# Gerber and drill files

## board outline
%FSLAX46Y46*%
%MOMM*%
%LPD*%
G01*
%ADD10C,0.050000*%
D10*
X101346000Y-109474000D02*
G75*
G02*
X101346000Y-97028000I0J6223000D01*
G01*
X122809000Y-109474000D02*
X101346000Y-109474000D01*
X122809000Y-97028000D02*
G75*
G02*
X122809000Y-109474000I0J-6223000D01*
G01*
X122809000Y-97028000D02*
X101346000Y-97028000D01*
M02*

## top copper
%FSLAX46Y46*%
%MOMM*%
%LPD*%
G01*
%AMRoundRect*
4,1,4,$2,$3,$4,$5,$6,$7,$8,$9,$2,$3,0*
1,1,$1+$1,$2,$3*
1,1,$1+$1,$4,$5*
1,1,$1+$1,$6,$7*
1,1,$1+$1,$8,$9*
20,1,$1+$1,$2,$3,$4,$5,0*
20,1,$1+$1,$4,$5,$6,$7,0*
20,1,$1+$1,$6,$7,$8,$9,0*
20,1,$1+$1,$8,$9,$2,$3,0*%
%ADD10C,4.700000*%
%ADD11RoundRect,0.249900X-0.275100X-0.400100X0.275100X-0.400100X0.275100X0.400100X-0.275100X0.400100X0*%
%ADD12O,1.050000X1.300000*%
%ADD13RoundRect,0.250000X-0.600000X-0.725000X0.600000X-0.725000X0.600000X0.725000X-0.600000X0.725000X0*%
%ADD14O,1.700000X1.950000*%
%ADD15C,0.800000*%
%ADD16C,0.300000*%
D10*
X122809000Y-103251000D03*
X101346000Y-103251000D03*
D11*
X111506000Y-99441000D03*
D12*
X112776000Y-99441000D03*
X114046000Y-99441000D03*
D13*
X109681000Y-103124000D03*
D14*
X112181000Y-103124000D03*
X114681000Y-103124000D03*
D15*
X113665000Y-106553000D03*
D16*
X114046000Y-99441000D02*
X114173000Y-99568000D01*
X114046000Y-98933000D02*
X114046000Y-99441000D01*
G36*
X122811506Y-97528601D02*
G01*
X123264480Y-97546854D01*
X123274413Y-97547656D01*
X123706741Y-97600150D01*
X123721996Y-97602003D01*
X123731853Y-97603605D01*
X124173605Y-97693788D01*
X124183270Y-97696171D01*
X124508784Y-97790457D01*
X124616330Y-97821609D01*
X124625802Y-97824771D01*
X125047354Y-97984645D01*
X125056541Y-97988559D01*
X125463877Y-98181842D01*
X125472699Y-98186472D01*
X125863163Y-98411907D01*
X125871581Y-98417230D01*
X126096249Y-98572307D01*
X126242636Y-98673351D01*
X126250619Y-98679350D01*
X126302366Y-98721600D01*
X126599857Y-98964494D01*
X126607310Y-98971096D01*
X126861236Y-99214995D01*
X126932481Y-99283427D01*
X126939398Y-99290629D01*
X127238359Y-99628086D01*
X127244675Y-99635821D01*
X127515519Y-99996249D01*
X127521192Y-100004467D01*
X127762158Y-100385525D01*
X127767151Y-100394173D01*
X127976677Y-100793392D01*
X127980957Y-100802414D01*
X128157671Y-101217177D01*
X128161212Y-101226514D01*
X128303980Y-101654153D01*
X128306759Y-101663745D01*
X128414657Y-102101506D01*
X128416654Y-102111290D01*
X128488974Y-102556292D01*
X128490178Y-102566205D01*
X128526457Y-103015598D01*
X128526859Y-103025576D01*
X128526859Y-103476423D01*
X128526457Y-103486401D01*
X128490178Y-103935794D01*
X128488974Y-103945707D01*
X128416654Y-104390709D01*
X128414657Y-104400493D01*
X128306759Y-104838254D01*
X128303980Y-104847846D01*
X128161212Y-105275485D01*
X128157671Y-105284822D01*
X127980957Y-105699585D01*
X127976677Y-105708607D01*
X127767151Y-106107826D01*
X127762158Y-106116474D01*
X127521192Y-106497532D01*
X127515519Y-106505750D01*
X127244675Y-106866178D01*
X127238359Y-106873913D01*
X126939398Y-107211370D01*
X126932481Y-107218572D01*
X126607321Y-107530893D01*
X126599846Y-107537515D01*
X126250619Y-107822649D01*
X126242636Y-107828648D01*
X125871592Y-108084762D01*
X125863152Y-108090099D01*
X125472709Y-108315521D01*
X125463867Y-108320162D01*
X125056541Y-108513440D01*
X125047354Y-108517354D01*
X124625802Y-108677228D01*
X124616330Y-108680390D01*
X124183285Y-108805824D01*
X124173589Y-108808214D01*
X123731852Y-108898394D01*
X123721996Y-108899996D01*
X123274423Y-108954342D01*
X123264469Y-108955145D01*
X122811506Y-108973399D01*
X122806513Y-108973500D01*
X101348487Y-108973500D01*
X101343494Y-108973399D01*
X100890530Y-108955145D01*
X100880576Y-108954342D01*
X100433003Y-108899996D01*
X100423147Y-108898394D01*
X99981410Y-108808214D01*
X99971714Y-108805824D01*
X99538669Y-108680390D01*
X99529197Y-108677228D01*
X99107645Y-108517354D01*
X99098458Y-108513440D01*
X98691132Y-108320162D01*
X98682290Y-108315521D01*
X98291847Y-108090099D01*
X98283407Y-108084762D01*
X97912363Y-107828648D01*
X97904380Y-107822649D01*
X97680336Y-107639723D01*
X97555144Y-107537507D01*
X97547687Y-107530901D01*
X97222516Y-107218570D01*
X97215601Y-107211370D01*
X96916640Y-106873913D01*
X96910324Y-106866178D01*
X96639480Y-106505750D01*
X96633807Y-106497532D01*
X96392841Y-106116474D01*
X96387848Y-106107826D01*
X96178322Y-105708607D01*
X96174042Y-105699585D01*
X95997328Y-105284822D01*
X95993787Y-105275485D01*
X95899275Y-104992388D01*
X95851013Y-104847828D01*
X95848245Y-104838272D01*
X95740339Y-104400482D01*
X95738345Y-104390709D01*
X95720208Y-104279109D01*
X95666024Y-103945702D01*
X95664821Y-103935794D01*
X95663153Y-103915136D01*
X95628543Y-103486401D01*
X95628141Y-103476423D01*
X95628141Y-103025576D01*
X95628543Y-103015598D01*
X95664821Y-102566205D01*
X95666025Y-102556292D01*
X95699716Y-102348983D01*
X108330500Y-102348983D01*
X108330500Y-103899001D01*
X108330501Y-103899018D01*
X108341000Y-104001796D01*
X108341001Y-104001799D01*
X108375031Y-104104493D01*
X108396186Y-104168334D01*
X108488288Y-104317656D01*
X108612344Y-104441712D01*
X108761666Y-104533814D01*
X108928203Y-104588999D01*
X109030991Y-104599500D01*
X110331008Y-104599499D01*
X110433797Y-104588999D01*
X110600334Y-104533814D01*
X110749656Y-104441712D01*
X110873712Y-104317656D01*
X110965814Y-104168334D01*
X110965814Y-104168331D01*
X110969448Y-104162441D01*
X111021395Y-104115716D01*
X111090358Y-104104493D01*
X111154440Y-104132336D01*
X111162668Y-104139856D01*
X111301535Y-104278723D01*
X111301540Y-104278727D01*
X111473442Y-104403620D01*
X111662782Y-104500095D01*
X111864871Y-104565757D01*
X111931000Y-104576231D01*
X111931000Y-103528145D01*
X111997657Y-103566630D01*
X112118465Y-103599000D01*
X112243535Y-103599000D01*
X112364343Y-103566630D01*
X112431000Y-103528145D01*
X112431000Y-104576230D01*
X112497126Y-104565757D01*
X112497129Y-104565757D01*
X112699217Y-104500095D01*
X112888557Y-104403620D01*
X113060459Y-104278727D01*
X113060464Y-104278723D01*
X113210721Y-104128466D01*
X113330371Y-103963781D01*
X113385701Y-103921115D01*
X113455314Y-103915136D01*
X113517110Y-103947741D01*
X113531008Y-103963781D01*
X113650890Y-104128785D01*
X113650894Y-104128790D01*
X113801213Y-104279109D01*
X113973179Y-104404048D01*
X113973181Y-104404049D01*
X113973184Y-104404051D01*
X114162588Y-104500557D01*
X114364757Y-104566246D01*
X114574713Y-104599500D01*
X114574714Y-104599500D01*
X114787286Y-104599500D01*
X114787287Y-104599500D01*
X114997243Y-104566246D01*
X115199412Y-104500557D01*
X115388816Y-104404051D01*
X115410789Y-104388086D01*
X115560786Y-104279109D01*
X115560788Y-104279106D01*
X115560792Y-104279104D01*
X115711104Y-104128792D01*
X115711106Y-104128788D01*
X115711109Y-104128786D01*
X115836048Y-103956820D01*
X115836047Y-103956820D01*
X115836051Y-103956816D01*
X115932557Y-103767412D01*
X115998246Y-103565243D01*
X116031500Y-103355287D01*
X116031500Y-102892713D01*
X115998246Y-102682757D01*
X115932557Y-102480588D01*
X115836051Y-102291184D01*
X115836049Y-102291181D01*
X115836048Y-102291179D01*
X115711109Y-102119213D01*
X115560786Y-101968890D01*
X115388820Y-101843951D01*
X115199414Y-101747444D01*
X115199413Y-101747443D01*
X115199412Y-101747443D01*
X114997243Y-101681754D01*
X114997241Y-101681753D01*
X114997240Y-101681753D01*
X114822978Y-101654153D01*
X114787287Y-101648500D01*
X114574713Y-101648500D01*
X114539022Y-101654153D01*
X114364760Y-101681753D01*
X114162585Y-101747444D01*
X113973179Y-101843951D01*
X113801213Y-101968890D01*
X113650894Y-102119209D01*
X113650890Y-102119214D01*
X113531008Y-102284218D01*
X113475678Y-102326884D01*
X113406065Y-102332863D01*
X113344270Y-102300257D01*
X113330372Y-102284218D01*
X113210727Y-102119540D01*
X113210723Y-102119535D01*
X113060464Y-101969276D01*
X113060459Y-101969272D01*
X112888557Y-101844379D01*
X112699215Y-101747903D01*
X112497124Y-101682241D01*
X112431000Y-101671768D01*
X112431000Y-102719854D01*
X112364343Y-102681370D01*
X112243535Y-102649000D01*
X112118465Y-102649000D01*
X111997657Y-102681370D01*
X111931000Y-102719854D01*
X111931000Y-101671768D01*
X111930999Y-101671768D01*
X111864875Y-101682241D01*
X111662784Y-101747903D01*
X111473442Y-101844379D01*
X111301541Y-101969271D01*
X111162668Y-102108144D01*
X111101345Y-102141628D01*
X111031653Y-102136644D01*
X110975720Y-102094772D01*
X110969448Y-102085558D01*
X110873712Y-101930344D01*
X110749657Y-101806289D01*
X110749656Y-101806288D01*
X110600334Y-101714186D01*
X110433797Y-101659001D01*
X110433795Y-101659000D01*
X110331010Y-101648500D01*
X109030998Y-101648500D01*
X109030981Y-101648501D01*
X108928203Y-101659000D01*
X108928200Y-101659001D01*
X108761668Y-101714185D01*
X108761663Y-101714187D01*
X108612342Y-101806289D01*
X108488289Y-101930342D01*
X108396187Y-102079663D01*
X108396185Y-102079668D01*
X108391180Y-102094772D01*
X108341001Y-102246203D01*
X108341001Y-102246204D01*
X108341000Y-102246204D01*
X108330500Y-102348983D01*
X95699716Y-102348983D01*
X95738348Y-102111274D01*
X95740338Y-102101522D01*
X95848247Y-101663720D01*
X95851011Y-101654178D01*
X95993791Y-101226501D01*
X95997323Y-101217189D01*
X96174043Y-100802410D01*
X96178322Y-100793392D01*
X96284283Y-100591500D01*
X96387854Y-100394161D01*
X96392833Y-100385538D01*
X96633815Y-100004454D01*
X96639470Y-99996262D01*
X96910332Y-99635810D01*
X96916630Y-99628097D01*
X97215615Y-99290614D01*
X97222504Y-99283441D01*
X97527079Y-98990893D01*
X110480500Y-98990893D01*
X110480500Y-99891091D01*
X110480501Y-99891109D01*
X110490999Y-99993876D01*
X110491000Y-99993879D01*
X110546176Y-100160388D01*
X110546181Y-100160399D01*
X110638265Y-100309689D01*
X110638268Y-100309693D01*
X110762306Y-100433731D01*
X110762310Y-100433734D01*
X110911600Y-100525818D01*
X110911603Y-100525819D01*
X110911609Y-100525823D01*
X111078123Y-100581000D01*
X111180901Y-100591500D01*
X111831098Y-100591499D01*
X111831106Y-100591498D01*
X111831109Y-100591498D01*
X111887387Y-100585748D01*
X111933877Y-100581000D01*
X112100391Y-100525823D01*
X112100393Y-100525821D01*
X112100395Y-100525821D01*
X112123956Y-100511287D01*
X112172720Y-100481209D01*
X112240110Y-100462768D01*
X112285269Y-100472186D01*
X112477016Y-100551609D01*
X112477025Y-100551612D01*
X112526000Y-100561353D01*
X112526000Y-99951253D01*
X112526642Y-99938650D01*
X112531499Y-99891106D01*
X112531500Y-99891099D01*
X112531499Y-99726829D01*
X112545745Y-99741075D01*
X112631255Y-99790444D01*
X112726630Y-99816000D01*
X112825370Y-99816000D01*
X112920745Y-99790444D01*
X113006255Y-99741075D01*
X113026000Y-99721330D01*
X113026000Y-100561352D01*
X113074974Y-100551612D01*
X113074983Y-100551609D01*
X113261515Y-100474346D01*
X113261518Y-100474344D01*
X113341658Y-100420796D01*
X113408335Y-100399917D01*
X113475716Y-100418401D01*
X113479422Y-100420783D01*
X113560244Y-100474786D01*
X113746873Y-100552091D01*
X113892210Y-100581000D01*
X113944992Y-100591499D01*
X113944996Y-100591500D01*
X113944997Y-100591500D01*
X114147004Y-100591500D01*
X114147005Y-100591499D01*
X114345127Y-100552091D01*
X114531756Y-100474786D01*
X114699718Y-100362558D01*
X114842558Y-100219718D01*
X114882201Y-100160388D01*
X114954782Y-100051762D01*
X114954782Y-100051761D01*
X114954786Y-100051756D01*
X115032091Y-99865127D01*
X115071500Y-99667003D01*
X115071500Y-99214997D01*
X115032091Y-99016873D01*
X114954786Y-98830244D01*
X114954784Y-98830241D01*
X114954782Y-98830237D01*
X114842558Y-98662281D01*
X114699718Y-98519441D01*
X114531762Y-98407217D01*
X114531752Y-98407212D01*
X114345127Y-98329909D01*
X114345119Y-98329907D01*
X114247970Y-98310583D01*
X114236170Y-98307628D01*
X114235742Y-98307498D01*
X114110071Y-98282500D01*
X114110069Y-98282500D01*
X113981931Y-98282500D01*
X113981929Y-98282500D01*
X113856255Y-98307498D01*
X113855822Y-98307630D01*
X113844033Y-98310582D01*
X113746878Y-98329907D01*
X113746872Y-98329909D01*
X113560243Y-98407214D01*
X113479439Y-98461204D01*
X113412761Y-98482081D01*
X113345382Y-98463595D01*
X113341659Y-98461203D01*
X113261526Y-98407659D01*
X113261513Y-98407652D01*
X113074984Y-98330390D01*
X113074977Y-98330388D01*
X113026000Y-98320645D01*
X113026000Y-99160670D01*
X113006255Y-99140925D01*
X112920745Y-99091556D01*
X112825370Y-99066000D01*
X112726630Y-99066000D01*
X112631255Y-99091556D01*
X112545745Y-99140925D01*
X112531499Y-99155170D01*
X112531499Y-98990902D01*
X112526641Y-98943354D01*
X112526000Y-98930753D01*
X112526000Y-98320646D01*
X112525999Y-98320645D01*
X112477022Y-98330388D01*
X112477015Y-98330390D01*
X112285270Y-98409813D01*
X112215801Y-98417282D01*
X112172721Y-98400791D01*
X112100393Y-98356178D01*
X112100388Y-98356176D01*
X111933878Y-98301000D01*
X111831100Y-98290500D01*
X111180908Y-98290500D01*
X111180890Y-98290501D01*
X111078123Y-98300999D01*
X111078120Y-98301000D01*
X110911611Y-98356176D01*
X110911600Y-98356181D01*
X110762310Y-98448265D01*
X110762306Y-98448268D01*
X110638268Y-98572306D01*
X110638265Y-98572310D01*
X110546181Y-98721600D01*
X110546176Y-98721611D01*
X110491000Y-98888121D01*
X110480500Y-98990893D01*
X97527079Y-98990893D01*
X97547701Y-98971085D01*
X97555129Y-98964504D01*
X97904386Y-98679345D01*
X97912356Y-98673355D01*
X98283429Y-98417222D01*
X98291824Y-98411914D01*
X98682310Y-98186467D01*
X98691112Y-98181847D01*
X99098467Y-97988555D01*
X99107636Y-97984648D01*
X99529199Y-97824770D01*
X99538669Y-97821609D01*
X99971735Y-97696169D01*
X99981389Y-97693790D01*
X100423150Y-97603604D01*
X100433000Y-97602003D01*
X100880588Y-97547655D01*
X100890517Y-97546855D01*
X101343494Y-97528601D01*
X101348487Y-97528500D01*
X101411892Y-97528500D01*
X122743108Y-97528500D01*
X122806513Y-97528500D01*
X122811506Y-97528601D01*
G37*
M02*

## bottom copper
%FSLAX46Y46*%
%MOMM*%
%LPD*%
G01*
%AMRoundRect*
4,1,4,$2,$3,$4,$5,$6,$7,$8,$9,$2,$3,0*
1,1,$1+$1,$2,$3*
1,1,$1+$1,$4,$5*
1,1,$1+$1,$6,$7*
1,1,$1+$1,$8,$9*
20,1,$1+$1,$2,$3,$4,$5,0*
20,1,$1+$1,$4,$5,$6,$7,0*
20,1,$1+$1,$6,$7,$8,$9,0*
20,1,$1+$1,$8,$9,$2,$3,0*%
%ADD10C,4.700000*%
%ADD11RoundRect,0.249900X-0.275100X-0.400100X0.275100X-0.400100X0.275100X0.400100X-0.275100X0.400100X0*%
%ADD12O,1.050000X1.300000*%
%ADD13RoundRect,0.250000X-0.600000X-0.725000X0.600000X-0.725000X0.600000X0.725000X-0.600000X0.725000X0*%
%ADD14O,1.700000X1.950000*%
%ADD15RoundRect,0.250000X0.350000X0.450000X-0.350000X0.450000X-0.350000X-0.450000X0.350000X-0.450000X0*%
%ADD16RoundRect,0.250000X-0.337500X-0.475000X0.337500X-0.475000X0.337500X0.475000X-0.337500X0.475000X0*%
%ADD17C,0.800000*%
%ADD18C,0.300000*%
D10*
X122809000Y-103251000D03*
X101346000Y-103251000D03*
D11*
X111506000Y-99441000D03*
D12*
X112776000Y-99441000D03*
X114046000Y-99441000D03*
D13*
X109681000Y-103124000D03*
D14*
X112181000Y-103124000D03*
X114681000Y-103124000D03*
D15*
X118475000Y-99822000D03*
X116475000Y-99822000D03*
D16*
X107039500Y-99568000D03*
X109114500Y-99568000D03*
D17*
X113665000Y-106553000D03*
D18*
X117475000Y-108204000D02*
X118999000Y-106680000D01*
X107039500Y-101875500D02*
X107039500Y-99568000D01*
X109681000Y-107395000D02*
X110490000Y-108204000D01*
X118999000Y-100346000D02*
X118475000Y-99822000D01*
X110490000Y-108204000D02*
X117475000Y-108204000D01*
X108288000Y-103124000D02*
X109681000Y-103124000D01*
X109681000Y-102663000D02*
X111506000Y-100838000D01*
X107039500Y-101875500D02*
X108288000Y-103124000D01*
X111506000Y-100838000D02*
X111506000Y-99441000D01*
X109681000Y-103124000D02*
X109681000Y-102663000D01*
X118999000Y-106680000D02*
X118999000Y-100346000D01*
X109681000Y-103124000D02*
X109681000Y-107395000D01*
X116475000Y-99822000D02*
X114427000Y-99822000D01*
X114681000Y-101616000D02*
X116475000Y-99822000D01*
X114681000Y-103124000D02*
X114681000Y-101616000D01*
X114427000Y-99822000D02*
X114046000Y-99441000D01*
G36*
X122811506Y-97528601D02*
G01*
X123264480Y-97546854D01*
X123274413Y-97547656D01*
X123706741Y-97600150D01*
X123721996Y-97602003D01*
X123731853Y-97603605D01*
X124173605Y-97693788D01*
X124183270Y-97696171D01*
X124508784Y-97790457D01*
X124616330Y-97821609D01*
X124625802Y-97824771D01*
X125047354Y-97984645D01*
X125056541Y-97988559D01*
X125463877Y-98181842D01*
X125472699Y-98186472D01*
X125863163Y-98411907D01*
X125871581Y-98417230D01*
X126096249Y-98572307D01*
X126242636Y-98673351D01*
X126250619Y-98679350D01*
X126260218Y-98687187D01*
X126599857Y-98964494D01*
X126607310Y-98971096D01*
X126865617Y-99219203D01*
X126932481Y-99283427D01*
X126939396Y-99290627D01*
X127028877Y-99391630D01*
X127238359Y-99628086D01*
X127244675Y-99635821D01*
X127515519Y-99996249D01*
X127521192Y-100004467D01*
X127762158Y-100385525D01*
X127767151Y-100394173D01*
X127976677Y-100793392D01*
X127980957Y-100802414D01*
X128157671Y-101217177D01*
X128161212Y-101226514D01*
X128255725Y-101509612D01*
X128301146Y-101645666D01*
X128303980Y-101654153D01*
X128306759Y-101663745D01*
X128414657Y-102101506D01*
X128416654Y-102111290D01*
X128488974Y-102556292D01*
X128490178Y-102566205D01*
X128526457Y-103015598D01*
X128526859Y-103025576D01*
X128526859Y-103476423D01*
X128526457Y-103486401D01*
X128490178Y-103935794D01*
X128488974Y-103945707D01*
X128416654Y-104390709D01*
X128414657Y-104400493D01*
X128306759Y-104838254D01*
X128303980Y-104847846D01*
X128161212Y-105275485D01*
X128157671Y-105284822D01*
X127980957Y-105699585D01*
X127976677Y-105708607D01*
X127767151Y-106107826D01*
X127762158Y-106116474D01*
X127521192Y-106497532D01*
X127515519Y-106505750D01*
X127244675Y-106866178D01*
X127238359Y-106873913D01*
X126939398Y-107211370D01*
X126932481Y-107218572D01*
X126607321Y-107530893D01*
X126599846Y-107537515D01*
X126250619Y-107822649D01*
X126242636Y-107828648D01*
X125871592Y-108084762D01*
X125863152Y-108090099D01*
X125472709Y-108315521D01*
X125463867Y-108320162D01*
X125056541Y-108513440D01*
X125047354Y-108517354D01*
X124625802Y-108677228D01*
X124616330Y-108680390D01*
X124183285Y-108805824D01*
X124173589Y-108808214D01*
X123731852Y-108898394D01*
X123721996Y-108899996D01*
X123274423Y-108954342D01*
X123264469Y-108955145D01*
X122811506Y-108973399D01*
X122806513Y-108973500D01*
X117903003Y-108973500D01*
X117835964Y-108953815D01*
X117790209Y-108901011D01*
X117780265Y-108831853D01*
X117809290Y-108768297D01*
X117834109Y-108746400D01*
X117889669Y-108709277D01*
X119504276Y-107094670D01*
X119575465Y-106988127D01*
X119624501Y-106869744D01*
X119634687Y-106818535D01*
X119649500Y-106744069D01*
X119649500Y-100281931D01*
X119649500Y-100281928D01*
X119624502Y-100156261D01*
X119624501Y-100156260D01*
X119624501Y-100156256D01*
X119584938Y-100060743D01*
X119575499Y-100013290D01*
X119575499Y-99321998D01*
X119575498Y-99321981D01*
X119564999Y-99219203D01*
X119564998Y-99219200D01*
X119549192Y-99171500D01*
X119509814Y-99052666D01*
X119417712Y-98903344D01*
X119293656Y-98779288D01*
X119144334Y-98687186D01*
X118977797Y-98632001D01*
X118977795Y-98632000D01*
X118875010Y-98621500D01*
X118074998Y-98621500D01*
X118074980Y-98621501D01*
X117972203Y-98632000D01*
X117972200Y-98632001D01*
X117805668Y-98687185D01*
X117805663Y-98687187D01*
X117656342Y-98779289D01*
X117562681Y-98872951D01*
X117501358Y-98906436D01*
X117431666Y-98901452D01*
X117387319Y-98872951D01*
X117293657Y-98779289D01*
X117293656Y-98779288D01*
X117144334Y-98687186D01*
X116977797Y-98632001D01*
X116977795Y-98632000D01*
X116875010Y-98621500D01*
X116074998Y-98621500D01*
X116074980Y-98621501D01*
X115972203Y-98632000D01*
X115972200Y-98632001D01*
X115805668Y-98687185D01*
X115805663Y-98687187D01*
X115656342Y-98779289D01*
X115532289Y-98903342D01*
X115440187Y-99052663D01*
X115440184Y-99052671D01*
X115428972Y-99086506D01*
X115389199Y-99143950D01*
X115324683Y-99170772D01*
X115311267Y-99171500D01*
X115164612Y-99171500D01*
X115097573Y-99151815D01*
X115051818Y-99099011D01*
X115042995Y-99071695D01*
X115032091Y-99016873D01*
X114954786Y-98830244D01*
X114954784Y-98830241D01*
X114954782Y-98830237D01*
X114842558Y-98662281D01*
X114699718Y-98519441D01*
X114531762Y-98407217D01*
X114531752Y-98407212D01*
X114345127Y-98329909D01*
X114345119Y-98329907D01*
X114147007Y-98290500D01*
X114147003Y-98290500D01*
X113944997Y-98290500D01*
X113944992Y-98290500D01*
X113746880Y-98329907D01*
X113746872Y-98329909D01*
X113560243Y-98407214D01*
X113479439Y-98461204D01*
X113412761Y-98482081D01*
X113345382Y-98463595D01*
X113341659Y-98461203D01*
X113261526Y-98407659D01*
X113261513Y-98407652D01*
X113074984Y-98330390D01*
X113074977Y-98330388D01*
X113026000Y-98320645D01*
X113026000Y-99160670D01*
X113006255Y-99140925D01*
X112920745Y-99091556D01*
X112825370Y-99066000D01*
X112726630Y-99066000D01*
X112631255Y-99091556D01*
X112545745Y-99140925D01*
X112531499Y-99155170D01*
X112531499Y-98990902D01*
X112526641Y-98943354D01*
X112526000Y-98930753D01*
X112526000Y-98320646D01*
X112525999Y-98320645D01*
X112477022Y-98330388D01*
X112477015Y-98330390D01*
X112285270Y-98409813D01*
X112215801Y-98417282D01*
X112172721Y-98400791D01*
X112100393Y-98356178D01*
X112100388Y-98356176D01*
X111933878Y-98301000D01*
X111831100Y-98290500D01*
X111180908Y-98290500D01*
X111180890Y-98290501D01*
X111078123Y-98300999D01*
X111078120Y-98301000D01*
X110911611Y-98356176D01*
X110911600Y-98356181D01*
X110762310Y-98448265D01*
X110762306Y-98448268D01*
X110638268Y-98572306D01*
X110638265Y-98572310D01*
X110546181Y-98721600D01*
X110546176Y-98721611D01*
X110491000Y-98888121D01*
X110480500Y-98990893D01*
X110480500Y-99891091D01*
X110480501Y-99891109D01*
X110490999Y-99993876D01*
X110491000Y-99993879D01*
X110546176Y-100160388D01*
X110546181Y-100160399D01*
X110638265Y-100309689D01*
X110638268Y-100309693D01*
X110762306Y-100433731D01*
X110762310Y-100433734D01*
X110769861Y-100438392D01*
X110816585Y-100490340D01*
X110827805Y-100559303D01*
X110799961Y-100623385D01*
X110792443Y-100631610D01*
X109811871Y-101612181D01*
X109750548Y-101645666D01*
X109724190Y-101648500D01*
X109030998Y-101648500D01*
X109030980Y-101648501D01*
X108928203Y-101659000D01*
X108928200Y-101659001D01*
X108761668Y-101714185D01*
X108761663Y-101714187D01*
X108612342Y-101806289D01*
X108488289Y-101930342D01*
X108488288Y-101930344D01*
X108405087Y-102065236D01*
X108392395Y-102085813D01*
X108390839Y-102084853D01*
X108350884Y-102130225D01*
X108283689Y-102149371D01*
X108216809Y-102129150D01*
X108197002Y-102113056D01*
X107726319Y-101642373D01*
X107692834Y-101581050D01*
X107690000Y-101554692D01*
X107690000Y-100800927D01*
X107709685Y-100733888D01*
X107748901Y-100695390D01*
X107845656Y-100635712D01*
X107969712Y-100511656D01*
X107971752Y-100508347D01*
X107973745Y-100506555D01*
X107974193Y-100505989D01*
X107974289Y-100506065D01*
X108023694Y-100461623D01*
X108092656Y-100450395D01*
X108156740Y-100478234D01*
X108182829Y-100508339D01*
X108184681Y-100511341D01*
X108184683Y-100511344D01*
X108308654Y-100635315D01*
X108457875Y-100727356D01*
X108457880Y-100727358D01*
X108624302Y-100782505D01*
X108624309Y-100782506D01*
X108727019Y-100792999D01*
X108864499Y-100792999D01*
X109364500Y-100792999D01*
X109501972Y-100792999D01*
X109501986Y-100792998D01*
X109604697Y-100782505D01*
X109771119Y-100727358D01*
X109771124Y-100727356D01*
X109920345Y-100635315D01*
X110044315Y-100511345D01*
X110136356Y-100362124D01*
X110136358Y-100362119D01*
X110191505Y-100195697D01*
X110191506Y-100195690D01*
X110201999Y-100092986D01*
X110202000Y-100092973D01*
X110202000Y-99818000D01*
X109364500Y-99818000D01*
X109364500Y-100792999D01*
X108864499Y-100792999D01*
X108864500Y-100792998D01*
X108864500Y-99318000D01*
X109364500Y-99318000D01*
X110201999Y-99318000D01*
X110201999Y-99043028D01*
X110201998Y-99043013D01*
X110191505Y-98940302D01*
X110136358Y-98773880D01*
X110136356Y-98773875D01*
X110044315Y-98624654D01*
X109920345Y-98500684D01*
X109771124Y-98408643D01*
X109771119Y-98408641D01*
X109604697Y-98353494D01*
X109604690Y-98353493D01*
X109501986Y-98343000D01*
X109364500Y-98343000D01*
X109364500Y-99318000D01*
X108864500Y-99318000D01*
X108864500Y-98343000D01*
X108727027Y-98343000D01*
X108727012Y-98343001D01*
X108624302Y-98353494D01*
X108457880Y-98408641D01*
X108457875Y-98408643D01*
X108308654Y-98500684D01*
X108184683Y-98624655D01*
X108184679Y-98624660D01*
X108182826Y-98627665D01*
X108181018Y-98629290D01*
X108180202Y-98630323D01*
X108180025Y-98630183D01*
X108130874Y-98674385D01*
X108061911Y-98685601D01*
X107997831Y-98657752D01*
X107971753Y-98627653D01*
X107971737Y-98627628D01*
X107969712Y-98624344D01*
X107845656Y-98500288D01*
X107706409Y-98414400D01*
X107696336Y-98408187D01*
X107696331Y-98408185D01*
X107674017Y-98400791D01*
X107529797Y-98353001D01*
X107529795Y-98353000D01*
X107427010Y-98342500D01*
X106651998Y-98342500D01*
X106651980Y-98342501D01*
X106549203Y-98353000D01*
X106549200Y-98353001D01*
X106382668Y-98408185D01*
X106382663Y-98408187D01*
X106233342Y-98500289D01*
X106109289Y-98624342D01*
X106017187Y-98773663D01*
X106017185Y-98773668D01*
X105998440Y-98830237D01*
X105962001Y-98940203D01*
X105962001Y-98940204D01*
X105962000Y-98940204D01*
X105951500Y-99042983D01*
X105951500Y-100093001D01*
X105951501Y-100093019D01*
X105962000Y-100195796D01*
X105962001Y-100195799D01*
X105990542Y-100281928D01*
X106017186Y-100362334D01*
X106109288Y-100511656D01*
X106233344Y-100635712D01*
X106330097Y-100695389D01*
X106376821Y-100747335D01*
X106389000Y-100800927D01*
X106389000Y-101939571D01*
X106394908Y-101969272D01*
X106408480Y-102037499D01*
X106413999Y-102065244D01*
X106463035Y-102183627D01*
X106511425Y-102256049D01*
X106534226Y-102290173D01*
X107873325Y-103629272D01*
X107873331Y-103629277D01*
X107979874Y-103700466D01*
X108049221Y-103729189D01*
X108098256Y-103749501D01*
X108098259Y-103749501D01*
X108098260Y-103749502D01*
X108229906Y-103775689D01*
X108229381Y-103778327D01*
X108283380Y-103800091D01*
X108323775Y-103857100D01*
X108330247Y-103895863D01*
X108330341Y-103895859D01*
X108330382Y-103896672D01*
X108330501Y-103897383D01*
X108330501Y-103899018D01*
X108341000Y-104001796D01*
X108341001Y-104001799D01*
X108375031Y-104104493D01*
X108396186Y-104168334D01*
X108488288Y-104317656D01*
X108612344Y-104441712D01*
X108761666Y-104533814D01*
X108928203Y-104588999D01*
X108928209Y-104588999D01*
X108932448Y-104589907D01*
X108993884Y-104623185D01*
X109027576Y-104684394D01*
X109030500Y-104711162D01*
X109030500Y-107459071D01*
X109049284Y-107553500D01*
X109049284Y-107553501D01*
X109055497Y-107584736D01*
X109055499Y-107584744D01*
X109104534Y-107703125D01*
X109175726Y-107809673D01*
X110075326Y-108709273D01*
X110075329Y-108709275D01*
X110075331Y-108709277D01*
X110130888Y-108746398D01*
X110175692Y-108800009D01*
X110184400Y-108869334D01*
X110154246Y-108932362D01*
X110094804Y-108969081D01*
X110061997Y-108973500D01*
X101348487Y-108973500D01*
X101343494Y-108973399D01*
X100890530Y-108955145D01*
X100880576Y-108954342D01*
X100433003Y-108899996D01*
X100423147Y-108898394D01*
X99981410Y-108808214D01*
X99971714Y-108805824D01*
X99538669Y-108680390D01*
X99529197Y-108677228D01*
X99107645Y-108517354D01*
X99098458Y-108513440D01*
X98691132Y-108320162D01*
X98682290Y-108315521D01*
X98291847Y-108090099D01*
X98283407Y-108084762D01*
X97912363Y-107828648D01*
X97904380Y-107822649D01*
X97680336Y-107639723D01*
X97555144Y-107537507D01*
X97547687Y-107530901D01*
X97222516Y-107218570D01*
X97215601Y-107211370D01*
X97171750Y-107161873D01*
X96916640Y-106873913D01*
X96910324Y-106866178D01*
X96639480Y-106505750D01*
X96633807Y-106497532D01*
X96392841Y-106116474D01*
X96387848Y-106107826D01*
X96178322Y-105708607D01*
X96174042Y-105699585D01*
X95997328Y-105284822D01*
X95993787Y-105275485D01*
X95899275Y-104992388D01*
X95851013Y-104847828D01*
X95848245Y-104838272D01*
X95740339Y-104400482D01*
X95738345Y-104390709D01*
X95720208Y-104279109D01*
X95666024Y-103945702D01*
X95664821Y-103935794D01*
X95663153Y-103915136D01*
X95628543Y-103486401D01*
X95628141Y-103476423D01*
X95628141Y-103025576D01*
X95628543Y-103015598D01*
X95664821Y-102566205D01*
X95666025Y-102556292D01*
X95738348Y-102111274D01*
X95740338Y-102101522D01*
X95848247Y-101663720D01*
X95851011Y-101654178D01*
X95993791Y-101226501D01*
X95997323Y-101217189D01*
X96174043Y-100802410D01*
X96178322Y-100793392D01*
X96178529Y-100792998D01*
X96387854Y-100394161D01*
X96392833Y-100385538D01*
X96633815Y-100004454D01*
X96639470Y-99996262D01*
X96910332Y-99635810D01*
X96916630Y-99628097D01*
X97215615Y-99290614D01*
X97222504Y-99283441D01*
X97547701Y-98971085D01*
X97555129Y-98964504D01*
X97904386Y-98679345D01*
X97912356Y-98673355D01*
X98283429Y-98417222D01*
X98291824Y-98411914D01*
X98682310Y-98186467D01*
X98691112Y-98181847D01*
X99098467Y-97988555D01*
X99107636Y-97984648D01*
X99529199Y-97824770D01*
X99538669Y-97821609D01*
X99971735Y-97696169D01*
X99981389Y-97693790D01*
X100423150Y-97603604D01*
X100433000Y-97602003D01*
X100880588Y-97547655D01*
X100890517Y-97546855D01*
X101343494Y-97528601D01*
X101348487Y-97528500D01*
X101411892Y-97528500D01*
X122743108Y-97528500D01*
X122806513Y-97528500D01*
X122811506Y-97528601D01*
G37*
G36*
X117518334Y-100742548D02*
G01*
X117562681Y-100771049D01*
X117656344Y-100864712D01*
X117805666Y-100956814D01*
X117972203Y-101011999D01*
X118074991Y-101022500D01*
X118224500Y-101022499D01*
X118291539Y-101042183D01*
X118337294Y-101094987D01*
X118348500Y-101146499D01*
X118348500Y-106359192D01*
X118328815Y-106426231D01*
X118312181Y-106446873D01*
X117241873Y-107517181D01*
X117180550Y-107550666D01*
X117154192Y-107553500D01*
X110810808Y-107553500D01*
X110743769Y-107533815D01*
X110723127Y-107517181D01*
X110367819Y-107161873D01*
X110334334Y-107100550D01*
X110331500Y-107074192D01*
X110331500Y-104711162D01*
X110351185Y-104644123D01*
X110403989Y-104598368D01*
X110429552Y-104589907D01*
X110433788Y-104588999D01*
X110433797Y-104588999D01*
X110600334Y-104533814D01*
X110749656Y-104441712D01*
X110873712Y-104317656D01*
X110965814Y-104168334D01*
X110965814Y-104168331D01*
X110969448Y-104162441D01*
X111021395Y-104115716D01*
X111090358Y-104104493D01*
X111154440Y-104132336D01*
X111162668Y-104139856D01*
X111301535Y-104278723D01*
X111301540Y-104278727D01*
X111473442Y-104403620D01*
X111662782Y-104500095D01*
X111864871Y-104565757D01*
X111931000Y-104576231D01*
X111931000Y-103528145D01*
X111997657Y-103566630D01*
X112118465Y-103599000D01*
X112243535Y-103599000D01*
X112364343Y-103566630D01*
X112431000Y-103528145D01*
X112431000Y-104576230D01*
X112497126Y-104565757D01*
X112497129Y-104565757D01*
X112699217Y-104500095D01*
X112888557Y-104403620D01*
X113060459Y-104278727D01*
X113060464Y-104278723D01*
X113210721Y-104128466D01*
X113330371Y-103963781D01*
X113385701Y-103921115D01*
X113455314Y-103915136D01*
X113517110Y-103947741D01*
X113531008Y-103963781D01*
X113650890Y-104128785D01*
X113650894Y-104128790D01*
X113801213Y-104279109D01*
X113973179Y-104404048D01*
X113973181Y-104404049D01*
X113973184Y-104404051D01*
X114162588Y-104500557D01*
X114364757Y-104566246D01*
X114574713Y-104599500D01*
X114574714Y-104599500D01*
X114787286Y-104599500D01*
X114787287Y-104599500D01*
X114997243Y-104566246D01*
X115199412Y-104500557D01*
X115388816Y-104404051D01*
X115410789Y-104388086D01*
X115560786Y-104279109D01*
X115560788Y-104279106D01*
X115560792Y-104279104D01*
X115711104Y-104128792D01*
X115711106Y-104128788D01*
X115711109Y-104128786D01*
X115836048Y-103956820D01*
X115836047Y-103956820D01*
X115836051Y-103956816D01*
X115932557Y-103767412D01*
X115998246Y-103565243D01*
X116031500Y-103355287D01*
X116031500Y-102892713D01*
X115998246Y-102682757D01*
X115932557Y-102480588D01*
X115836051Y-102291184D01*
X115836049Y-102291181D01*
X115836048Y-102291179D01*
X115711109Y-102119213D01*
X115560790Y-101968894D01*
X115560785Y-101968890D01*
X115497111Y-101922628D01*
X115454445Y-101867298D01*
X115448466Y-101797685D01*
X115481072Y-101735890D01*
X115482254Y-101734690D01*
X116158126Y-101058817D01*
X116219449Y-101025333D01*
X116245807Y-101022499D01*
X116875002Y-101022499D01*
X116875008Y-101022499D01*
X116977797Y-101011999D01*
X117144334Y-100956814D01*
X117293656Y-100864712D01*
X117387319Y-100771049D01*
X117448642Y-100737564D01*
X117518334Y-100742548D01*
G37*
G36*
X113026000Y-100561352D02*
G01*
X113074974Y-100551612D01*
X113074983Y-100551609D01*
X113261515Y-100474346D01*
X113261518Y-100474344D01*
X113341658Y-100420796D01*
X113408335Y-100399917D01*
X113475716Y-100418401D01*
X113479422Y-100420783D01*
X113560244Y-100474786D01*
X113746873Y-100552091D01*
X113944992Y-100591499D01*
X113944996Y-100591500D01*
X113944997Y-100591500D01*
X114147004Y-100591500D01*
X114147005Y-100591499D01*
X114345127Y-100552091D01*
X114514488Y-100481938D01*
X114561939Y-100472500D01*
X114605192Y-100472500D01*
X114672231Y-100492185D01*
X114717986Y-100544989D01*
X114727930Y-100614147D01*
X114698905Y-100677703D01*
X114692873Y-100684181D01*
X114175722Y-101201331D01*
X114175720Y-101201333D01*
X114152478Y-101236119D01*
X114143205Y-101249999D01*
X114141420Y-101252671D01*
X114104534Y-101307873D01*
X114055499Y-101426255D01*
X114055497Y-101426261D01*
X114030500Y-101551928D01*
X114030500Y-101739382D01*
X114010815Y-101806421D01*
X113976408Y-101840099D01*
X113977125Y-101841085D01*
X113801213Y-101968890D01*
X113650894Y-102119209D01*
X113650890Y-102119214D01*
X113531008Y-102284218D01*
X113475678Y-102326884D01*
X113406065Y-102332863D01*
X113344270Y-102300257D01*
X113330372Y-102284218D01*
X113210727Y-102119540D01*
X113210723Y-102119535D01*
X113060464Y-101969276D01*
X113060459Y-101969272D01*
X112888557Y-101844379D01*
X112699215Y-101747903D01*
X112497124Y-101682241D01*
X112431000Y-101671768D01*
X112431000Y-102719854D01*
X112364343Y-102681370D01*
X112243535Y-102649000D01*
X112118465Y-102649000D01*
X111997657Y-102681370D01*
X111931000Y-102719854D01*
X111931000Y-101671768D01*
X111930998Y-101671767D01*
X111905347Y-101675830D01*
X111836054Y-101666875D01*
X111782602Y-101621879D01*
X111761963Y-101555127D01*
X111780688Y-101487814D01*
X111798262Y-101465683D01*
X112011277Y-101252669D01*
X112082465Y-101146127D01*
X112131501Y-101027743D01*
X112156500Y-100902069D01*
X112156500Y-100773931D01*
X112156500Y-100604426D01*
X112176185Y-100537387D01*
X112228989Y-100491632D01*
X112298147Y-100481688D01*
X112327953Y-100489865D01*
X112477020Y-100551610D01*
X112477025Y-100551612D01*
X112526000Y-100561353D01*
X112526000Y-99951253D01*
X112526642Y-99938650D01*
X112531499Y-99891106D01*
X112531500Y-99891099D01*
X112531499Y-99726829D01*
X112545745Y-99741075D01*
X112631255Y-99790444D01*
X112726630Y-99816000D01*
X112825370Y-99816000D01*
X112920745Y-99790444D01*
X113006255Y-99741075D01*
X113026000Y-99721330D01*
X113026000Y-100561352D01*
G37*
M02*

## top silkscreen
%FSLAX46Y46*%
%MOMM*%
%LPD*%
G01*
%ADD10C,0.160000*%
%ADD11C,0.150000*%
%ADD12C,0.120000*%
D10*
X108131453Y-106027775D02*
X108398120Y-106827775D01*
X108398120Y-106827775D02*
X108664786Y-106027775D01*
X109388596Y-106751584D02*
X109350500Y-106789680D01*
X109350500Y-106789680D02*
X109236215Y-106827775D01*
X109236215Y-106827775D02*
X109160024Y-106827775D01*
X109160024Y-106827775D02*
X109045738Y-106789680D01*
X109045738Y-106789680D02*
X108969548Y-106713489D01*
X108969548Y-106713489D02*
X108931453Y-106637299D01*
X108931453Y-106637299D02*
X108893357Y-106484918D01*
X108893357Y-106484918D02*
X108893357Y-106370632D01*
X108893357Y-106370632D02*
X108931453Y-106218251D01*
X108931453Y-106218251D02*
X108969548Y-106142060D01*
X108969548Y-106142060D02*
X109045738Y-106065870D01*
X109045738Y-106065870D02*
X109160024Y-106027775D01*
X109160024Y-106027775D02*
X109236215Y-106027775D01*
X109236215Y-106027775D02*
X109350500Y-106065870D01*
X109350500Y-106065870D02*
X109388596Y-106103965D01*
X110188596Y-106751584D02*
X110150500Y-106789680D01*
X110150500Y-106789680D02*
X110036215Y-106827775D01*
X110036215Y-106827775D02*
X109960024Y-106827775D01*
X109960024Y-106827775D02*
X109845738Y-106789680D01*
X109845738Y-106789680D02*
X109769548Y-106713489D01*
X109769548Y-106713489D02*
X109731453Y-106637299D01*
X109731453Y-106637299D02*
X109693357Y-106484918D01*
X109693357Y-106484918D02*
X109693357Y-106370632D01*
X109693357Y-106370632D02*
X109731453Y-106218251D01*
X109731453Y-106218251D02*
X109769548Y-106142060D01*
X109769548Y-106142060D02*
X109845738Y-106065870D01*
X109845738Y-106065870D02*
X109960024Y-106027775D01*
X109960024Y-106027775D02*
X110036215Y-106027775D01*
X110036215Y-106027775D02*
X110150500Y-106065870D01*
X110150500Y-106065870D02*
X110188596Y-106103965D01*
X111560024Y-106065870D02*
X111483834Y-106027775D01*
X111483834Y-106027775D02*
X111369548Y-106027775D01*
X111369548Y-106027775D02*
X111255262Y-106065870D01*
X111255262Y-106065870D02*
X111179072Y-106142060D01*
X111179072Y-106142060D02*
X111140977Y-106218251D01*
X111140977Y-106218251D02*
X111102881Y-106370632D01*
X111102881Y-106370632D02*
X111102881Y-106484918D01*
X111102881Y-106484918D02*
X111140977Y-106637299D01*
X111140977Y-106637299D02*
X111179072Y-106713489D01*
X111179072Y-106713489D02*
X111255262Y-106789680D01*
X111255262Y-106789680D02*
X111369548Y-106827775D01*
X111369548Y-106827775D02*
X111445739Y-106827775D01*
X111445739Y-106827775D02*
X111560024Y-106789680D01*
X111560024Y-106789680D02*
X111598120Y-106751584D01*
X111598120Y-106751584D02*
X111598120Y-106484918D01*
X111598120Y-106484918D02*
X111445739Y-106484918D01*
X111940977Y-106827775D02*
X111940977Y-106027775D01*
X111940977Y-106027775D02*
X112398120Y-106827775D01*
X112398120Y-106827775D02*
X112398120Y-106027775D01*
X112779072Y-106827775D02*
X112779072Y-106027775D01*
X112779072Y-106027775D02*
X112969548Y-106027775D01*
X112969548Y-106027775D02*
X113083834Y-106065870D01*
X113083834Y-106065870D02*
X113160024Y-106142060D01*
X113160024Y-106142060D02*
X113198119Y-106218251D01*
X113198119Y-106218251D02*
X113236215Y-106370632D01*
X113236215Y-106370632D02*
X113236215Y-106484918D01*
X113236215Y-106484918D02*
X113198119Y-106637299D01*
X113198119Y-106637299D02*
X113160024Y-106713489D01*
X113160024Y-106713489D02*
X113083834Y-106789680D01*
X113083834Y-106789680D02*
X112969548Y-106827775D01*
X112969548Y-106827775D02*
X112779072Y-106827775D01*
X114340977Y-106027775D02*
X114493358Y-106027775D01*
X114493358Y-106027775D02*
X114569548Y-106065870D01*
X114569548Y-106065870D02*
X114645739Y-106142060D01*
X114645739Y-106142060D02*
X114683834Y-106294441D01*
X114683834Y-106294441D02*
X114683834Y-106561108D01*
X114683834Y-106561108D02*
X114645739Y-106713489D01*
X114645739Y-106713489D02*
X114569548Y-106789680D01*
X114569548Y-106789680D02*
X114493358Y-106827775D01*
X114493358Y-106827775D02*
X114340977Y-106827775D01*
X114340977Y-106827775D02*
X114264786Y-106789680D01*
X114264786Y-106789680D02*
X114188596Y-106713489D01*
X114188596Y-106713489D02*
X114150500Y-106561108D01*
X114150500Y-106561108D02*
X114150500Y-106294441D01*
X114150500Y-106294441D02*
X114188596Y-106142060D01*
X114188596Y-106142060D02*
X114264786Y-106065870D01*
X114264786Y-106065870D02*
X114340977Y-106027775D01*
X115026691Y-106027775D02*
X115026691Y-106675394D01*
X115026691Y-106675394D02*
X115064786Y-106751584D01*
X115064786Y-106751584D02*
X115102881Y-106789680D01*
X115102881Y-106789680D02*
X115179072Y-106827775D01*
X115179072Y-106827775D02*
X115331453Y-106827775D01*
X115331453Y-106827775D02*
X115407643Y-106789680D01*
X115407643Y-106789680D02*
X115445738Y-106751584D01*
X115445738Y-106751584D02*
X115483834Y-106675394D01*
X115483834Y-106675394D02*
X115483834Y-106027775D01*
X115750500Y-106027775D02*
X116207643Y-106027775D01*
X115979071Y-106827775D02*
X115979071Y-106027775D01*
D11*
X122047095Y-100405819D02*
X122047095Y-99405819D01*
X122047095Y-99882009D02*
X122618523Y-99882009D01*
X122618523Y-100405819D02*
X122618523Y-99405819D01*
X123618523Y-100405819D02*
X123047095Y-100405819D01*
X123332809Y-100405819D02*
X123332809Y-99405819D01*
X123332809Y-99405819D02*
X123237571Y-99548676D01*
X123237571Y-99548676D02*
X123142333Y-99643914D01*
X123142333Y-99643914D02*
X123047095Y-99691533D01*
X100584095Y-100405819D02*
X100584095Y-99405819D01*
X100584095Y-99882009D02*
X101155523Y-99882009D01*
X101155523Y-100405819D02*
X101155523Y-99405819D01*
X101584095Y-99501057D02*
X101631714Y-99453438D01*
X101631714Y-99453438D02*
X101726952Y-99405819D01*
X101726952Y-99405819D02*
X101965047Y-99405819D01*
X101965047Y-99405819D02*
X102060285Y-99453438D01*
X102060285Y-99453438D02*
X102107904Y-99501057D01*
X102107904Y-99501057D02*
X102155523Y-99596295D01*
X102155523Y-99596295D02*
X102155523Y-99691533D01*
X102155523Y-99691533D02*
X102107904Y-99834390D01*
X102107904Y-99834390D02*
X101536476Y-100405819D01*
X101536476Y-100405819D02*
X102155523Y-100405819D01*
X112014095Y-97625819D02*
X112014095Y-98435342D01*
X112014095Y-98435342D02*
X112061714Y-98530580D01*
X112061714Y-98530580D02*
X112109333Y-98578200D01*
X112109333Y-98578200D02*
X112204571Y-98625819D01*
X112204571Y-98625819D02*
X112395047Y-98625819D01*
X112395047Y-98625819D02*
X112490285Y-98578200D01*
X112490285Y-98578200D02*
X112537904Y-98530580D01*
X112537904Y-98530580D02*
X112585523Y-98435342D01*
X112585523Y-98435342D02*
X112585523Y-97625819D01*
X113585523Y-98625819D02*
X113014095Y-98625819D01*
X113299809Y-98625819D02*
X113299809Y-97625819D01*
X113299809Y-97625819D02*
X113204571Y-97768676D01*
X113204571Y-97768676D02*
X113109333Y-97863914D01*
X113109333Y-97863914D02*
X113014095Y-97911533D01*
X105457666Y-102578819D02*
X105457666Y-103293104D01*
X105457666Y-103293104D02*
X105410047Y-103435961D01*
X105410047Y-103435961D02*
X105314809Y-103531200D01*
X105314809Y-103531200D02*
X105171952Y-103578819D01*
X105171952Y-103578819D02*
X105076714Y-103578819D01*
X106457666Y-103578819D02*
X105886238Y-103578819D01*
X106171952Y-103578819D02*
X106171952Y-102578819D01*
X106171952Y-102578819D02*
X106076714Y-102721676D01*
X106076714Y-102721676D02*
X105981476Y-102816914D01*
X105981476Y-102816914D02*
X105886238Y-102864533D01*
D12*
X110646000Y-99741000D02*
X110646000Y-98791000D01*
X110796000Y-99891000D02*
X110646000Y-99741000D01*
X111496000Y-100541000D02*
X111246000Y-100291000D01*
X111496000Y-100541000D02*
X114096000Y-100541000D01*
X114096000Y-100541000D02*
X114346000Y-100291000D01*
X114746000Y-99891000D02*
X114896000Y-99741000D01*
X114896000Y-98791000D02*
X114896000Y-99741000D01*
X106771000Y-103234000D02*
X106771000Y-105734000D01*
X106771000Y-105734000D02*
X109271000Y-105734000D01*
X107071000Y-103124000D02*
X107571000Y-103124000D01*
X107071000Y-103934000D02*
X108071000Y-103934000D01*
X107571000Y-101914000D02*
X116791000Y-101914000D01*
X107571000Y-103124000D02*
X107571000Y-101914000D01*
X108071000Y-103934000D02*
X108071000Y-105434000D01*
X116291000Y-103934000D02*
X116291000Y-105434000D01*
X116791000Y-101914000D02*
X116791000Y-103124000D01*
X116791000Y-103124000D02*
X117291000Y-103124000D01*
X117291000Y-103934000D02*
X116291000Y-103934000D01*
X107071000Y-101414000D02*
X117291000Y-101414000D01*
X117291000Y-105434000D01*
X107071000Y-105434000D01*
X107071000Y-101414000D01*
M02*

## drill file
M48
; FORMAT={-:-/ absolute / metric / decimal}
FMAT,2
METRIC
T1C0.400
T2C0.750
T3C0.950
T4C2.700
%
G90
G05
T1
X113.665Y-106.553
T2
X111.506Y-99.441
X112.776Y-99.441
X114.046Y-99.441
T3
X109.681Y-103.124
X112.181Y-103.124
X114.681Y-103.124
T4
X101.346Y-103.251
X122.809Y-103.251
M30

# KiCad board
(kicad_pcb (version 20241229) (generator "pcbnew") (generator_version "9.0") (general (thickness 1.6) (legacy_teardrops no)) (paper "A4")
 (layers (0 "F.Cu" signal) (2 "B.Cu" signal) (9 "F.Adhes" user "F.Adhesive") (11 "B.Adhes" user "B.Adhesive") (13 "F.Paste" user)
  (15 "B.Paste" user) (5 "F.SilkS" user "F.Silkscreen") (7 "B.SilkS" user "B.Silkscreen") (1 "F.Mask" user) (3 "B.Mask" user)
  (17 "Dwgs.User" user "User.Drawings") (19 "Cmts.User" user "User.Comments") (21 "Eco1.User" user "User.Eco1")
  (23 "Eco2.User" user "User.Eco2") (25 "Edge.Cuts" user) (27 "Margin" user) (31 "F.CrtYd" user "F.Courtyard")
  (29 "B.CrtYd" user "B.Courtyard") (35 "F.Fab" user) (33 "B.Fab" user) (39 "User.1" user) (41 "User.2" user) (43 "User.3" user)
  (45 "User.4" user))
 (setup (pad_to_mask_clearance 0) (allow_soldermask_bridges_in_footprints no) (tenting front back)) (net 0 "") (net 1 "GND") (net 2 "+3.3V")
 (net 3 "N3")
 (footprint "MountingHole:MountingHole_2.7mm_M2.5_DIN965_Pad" (layer "F.Cu") (at 122.809 103.251)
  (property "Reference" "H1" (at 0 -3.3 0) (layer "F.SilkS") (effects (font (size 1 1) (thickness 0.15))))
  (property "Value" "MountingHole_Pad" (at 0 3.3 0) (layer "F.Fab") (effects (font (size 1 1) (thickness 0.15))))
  (pad "1" thru_hole circle (at 0 0) (size 4.7 4.7) (drill 2.7) (layers "*.Cu" "*.Mask") (remove_unused_layers no) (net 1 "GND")
   (zone_connect 2)))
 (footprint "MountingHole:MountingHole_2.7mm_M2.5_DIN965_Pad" (layer "F.Cu") (at 101.346 103.251)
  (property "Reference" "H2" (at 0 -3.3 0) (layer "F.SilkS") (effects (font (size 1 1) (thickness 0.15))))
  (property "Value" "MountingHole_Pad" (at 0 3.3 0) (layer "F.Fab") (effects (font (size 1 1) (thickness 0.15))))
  (pad "1" thru_hole circle (at 0 0) (size 4.7 4.7) (drill 2.7) (layers "*.Cu" "*.Mask") (remove_unused_layers no) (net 1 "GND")
   (zone_connect 2)))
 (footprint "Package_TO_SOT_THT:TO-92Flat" (layer "F.Cu") (at 111.506 99.441)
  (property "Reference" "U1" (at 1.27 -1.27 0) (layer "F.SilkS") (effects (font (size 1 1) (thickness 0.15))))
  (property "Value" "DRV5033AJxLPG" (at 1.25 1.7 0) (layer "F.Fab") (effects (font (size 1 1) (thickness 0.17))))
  (fp_line (start -0.86 0.3) (end -0.86 -0.65) (stroke (width 0.12) (type solid)) (layer "F.SilkS"))
  (fp_line (start -0.71 0.45) (end -0.86 0.3) (stroke (width 0.12) (type solid)) (layer "F.SilkS"))
  (fp_line (start -0.01 1.1) (end -0.26 0.85) (stroke (width 0.12) (type solid)) (layer "F.SilkS"))
  (fp_line (start -0.01 1.1) (end 2.59 1.1) (stroke (width 0.12) (type solid)) (layer "F.SilkS"))
  (fp_line (start 2.59 1.1) (end 2.84 0.85) (stroke (width 0.12) (type solid)) (layer "F.SilkS"))
  (fp_line (start 3.24 0.45) (end 3.39 0.3) (stroke (width 0.12) (type solid)) (layer "F.SilkS"))
  (fp_line (start 3.39 -0.65) (end 3.39 0.3) (stroke (width 0.12) (type solid)) (layer "F.SilkS"))
  (pad "1" thru_hole roundrect (at 0 0) (size 1.05 1.3) (drill 0.75) (layers "*.Cu" "*.Mask") (remove_unused_layers no)
   (roundrect_rratio 0.238) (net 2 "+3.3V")
   (teardrops (best_length_ratio 0.5) (max_length 1) (best_width_ratio 1) (max_width 1) (curved_edges no) (filter_ratio 0.9) (enabled no)
    (allow_two_segments yes) (prefer_zone_connections yes)))
  (pad "2" thru_hole oval (at 1.27 0) (size 1.05 1.3) (drill 0.75) (layers "*.Cu" "*.Mask") (remove_unused_layers no) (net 1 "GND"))
  (pad "3" thru_hole oval (at 2.54 0) (size 1.05 1.3) (drill 0.75) (layers "*.Cu" "*.Mask") (remove_unused_layers no) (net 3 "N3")))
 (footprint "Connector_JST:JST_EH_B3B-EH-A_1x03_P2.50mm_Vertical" (layer "F.Cu") (at 109.681 103.124)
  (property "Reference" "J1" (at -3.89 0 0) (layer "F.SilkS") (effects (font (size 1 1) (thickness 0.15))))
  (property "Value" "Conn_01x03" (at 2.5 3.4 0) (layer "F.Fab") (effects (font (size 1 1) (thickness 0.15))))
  (fp_line (start -2.91 0.11) (end -2.91 2.61) (stroke (width 0.12) (type solid)) (layer "F.SilkS"))
  (fp_line (start -2.91 2.61) (end -0.41 2.61) (stroke (width 0.12) (type solid)) (layer "F.SilkS"))
  (fp_line (start -2.61 0) (end -2.11 0) (stroke (width 0.12) (type solid)) (layer "F.SilkS"))
  (fp_line (start -2.61 0.81) (end -1.61 0.81) (stroke (width 0.12) (type solid)) (layer "F.SilkS"))
  (fp_line (start -2.11 -1.21) (end 7.11 -1.21) (stroke (width 0.12) (type solid)) (layer "F.SilkS"))
  (fp_line (start -2.11 0) (end -2.11 -1.21) (stroke (width 0.12) (type solid)) (layer "F.SilkS"))
  (fp_line (start -1.61 0.81) (end -1.61 2.31) (stroke (width 0.12) (type solid)) (layer "F.SilkS"))
  (fp_line (start 6.61 0.81) (end 6.61 2.31) (stroke (width 0.12) (type solid)) (layer "F.SilkS"))
  (fp_line (start 7.11 -1.21) (end 7.11 0) (stroke (width 0.12) (type solid)) (layer "F.SilkS"))
  (fp_line (start 7.11 0) (end 7.61 0) (stroke (width 0.12) (type solid)) (layer "F.SilkS"))
  (fp_line (start 7.61 0.81) (end 6.61 0.81) (stroke (width 0.12) (type solid)) (layer "F.SilkS"))
  (fp_rect (start -2.61 -1.71) (end 7.61 2.31) (stroke (width 0.12) (type solid)) (fill no) (layer "F.SilkS"))
  (pad "1" thru_hole roundrect (at 0 0) (size 1.7 1.95) (drill 0.95) (layers "*.Cu" "*.Mask") (remove_unused_layers no)
   (roundrect_rratio 0.147059) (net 2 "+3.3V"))
  (pad "2" thru_hole oval (at 2.5 0) (size 1.7 1.95) (drill 0.95) (layers "*.Cu" "*.Mask") (remove_unused_layers no) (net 1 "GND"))
  (pad "3" thru_hole oval (at 5 0) (size 1.7 1.95) (drill 0.95) (layers "*.Cu" "*.Mask") (remove_unused_layers no) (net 3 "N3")))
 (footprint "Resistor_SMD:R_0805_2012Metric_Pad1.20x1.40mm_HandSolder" (layer "B.Cu") (at 117.475 99.822 180)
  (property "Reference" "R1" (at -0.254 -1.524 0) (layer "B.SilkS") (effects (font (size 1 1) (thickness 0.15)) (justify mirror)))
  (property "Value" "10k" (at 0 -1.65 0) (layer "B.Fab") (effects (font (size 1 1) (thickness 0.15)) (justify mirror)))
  (pad "1" smd roundrect (at -1 0 180) (size 1.2 1.4) (layers "B.Cu" "B.Mask" "B.Paste") (roundrect_rratio 0.208333) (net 2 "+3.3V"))
  (pad "2" smd roundrect (at 1 0 180) (size 1.2 1.4) (layers "B.Cu" "B.Mask" "B.Paste") (roundrect_rratio 0.208333) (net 3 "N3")))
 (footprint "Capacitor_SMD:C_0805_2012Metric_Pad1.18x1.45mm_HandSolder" (layer "B.Cu") (at 108.077 99.568)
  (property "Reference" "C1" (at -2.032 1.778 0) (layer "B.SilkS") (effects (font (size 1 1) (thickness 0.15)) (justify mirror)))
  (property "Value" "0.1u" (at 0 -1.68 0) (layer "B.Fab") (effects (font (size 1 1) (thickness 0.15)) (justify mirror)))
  (pad "1" smd roundrect (at -1.0375 0) (size 1.175 1.45) (layers "B.Cu" "B.Mask" "B.Paste") (roundrect_rratio 0.212766) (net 2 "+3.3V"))
  (pad "2" smd roundrect (at 1.0375 0) (size 1.175 1.45) (layers "B.Cu" "B.Mask" "B.Paste") (roundrect_rratio 0.212766) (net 1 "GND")))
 (gr_arc (start 101.346 109.474) (mid 95.123 103.251) (end 101.346 97.028) (stroke (width 0.05) (type default)) (layer "Edge.Cuts"))
 (gr_line (start 122.809 109.474) (end 101.346 109.474) (stroke (width 0.05) (type default)) (layer "Edge.Cuts"))
 (gr_arc (start 122.809 97.028) (mid 129.032 103.251) (end 122.809 109.474) (stroke (width 0.05) (type default)) (layer "Edge.Cuts"))
 (gr_line (start 122.809 97.028) (end 101.346 97.028) (stroke (width 0.05) (type default)) (layer "Edge.Cuts"))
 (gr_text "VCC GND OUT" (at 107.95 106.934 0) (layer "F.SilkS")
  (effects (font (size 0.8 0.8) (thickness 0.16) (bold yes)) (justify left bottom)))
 (via (at 113.665 106.553) (size 0.8) (drill 0.4) (layers "F.Cu" "B.Cu") (free yes) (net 1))
 (segment (start 117.475 108.204) (end 118.999 106.68) (width 0.3) (layer "B.Cu") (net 2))
 (segment (start 107.0395 101.8755) (end 107.0395 99.568) (width 0.3) (layer "B.Cu") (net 2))
 (segment (start 109.681 107.395) (end 110.49 108.204) (width 0.3) (layer "B.Cu") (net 2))
 (segment (start 118.999 100.346) (end 118.475 99.822) (width 0.3) (layer "B.Cu") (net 2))
 (segment (start 110.49 108.204) (end 117.475 108.204) (width 0.3) (layer "B.Cu") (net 2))
 (segment (start 108.288 103.124) (end 109.681 103.124) (width 0.3) (layer "B.Cu") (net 2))
 (segment (start 109.681 102.663) (end 111.506 100.838) (width 0.3) (layer "B.Cu") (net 2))
 (segment (start 107.0395 101.8755) (end 108.288 103.124) (width 0.3) (layer "B.Cu") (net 2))
 (segment (start 111.506 100.838) (end 111.506 99.441) (width 0.3) (layer "B.Cu") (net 2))
 (segment (start 109.681 103.124) (end 109.681 102.663) (width 0.3) (layer "B.Cu") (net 2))
 (segment (start 118.999 106.68) (end 118.999 100.346) (width 0.3) (layer "B.Cu") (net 2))
 (segment (start 109.681 103.124) (end 109.681 107.395) (width 0.3) (layer "B.Cu") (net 2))
 (segment (start 114.046 99.441) (end 114.173 99.568) (width 0.3) (layer "F.Cu") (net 3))
 (segment (start 114.046 98.933) (end 114.046 99.441) (width 0.3) (layer "F.Cu") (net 3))
 (segment (start 116.475 99.822) (end 114.427 99.822) (width 0.3) (layer "B.Cu") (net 3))
 (segment (start 114.681 101.616) (end 116.475 99.822) (width 0.3) (layer "B.Cu") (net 3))
 (segment (start 114.681 103.124) (end 114.681 101.616) (width 0.3) (layer "B.Cu") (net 3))
 (segment (start 114.427 99.822) (end 114.046 99.441) (width 0.3) (layer "B.Cu") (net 3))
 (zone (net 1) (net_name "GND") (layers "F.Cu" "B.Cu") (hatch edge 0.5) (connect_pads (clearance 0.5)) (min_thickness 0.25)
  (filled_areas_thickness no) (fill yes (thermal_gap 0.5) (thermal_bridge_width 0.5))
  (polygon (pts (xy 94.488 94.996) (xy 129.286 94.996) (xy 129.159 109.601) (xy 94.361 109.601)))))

